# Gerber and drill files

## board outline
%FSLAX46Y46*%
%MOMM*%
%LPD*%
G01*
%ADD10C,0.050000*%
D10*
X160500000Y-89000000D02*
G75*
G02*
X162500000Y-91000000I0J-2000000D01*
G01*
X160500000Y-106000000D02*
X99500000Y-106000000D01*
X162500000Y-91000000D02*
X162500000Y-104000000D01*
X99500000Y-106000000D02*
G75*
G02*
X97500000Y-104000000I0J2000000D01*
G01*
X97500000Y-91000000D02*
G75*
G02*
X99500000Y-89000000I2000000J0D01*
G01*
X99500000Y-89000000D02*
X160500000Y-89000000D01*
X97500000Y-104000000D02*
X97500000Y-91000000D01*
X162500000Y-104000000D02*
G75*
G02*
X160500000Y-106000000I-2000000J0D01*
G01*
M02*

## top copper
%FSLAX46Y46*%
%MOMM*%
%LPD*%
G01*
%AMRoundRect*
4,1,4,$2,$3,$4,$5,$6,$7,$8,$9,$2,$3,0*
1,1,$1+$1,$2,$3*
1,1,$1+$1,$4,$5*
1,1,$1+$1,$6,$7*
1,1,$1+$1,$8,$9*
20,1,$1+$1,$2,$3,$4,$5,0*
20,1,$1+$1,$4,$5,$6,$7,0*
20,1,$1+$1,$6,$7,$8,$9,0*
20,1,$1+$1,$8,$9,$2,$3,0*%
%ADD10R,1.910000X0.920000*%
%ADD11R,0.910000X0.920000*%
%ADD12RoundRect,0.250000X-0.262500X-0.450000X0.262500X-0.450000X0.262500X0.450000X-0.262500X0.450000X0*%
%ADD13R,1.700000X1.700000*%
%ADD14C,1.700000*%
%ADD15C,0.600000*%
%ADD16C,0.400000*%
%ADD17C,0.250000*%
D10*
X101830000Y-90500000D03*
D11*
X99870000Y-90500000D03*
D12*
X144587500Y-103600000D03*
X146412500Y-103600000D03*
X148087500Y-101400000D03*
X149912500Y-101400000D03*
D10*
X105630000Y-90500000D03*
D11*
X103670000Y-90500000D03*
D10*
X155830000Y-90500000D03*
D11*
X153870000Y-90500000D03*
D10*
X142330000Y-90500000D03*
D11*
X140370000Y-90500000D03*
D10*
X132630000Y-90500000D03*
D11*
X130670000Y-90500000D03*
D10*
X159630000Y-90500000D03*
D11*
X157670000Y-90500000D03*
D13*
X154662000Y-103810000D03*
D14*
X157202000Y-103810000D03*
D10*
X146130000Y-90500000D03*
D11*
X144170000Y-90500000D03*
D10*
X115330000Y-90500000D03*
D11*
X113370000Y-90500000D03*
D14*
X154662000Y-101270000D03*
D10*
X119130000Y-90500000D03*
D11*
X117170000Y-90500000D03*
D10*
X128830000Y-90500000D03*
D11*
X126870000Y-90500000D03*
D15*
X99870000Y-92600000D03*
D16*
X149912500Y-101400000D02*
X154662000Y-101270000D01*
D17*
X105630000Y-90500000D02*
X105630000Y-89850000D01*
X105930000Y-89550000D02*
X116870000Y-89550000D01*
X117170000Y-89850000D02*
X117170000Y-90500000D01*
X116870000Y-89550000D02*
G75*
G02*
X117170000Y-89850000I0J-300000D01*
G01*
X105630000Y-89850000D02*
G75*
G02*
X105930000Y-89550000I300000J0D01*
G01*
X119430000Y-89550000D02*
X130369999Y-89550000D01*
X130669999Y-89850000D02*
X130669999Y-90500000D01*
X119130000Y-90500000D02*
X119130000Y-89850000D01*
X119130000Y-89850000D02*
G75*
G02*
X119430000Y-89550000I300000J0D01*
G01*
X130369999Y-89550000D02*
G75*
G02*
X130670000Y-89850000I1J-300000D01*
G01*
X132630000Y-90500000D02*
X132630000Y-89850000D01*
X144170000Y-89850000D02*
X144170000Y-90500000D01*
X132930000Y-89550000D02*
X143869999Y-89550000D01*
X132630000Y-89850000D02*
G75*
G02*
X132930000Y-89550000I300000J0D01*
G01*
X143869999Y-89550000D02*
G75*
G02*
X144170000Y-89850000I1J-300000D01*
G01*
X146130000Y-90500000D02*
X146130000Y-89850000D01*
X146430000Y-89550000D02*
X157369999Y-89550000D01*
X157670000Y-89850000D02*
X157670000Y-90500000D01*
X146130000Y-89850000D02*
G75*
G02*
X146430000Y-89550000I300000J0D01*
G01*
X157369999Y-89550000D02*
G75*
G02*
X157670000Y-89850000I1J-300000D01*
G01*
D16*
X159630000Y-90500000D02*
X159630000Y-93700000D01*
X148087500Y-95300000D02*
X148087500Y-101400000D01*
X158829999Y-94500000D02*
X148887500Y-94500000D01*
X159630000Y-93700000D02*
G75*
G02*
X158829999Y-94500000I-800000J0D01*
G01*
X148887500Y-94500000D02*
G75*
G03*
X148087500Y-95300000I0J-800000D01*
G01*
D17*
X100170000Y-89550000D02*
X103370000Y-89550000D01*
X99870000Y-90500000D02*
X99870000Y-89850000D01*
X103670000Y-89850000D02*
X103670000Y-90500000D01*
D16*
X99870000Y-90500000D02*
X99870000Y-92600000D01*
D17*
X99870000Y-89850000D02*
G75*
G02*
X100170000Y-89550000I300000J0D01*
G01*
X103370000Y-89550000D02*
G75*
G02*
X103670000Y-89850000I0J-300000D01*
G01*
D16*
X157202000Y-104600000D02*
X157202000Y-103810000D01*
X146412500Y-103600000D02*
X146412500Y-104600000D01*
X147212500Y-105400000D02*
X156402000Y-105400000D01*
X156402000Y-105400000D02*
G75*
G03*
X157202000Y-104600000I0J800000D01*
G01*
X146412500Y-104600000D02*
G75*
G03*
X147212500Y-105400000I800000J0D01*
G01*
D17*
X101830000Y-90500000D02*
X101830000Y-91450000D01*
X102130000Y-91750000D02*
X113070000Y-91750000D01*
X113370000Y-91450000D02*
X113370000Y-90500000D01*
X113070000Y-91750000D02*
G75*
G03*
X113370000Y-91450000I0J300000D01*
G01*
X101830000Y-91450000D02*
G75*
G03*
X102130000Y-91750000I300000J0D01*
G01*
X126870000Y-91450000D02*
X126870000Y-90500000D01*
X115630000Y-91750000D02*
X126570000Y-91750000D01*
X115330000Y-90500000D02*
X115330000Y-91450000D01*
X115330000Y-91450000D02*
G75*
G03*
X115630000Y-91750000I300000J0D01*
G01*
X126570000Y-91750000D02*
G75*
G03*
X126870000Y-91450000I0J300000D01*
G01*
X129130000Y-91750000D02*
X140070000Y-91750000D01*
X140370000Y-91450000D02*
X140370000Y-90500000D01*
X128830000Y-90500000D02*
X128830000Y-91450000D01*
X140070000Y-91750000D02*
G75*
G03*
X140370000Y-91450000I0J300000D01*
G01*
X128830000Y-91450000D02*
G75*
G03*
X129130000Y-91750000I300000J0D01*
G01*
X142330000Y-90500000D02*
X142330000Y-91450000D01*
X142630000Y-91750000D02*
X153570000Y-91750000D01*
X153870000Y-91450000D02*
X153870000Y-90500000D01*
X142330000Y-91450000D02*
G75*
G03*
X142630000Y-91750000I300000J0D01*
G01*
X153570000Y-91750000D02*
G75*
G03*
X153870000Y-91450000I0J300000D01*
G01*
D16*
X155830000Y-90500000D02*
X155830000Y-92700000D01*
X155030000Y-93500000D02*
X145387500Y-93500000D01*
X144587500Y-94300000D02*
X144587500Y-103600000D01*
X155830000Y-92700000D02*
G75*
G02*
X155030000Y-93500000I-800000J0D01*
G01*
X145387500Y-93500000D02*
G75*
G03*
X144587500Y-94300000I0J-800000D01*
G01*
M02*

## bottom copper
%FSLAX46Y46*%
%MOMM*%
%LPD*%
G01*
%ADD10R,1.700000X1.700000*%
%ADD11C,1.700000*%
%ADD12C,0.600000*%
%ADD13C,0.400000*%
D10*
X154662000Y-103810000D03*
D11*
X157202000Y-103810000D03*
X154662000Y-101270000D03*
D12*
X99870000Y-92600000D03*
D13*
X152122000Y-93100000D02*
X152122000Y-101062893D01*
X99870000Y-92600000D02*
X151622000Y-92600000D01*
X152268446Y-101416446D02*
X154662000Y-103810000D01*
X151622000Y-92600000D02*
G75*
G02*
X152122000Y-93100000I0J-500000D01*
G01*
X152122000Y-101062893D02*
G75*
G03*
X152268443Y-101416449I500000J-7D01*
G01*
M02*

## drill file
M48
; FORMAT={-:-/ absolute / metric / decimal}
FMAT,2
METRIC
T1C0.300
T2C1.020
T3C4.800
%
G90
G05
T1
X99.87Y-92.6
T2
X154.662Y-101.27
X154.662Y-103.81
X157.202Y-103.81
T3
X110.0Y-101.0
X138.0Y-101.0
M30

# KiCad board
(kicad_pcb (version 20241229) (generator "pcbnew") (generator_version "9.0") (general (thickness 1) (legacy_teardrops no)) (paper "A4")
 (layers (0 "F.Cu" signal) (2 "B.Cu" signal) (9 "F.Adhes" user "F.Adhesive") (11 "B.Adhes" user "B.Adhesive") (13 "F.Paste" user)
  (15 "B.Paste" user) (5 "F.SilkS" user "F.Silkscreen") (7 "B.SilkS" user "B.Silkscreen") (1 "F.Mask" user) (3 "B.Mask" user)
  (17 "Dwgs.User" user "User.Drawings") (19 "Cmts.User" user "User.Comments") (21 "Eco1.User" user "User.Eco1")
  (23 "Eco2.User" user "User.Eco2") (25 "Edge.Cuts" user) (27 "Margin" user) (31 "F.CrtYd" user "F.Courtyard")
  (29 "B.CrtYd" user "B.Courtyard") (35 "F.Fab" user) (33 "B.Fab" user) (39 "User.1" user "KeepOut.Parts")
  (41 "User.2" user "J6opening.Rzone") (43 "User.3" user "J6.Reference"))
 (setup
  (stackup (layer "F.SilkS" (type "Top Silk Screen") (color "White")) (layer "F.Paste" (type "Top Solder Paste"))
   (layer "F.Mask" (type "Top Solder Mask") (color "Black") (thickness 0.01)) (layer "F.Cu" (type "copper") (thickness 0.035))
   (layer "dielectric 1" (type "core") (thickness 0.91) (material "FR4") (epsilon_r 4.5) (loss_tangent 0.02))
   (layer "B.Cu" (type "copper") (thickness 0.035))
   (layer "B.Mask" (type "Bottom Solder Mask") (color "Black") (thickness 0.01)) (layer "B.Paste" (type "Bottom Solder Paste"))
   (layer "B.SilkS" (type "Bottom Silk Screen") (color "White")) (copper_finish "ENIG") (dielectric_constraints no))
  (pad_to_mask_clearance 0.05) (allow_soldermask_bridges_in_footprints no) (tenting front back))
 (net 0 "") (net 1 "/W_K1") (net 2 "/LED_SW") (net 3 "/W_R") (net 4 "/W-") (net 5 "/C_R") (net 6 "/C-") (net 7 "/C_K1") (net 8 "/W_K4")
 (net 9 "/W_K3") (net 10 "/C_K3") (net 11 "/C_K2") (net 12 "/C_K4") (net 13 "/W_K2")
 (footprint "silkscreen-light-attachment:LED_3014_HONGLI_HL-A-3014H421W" (layer "F.Cu") (at 101.1 90.5 180)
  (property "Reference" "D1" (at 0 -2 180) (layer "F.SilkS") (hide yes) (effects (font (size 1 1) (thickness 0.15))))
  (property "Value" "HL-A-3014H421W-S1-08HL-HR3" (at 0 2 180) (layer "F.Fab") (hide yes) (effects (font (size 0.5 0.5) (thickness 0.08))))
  (pad "1" smd rect (at -0.73 0 180) (size 1.91 0.92) (layers "F.Cu" "F.Mask" "F.Paste") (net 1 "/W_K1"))
  (pad "2" smd rect (at 1.23 0 180) (size 0.91 0.92) (layers "F.Cu" "F.Mask" "F.Paste") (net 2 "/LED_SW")))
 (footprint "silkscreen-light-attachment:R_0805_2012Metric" (layer "F.Cu") (at 145.5 103.6)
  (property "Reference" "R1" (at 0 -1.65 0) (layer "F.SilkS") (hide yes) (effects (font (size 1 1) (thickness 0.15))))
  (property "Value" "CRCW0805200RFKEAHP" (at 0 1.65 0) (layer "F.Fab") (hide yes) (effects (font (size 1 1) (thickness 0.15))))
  (pad "1" smd roundrect (at -0.9125 0) (size 1.025 1.4) (layers "F.Cu" "F.Mask" "F.Paste") (roundrect_rratio 0.243902) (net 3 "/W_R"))
  (pad "2" smd roundrect (at 0.9125 0) (size 1.025 1.4) (layers "F.Cu" "F.Mask" "F.Paste") (roundrect_rratio 0.243902) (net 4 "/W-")))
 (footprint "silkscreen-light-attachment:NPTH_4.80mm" (layer "F.Cu") (at 110 101)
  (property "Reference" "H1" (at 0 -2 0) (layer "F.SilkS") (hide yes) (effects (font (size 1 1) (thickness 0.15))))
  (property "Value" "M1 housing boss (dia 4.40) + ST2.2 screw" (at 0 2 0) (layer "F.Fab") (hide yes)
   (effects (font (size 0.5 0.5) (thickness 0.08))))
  (pad "" np_thru_hole circle (at 0 0) (size 4.8 4.8) (drill 4.8) (layers "*.Cu" "*.Mask")))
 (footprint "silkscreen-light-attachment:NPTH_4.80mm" (layer "F.Cu") (at 138 101)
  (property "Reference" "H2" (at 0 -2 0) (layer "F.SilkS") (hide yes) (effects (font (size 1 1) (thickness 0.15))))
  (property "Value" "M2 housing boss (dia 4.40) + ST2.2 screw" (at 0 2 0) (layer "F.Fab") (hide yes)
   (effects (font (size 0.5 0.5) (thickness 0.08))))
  (pad "" np_thru_hole circle (at 0 0) (size 4.8 4.8) (drill 4.8) (layers "*.Cu" "*.Mask")))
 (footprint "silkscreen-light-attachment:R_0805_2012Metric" (layer "F.Cu") (at 149 101.4)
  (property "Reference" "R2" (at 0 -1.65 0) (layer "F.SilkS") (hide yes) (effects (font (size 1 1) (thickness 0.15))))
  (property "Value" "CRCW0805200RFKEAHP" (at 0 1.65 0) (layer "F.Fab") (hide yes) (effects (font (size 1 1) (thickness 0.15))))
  (pad "1" smd roundrect (at -0.9125 0) (size 1.025 1.4) (layers "F.Cu" "F.Mask" "F.Paste") (roundrect_rratio 0.243902) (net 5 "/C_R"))
  (pad "2" smd roundrect (at 0.9125 0) (size 1.025 1.4) (layers "F.Cu" "F.Mask" "F.Paste") (roundrect_rratio 0.243902) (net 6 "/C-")))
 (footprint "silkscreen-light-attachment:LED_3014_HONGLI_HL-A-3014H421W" (layer "F.Cu") (at 104.9 90.5 180)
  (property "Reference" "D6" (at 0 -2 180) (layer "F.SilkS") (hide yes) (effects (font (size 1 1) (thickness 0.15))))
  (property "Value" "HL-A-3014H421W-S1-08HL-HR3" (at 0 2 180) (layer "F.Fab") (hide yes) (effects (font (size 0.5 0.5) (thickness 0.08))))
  (pad "1" smd rect (at -0.73 0 180) (size 1.91 0.92) (layers "F.Cu" "F.Mask" "F.Paste") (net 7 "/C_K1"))
  (pad "2" smd rect (at 1.23 0 180) (size 0.91 0.92) (layers "F.Cu" "F.Mask" "F.Paste") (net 2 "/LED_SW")))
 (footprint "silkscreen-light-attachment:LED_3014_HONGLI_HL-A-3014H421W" (layer "F.Cu") (at 155.1 90.5 180)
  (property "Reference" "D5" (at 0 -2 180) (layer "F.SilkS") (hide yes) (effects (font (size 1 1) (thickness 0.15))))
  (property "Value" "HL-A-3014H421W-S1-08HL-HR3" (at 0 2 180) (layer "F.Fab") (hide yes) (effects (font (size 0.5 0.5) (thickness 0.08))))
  (pad "1" smd rect (at -0.73 0 180) (size 1.91 0.92) (layers "F.Cu" "F.Mask" "F.Paste") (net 3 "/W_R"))
  (pad "2" smd rect (at 1.23 0 180) (size 0.91 0.92) (layers "F.Cu" "F.Mask" "F.Paste") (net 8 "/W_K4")))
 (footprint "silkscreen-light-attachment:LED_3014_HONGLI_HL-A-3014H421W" (layer "F.Cu") (at 141.6 90.5 180)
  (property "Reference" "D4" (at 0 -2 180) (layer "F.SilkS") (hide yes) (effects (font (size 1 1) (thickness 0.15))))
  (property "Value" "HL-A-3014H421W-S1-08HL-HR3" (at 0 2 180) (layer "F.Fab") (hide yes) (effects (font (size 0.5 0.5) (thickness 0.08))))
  (pad "1" smd rect (at -0.73 0 180) (size 1.91 0.92) (layers "F.Cu" "F.Mask" "F.Paste") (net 8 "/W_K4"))
  (pad "2" smd rect (at 1.23 0 180) (size 0.91 0.92) (layers "F.Cu" "F.Mask" "F.Paste") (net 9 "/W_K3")))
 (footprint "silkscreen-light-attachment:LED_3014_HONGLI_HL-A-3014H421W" (layer "F.Cu") (at 131.9 90.5 180)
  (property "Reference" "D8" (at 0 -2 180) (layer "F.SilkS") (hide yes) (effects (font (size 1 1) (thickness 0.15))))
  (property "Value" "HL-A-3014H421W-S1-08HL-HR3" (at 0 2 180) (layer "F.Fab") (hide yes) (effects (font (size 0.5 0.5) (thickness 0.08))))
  (pad "1" smd rect (at -0.73 0 180) (size 1.91 0.92) (layers "F.Cu" "F.Mask" "F.Paste") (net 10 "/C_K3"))
  (pad "2" smd rect (at 1.23 0 180) (size 0.91 0.92) (layers "F.Cu" "F.Mask" "F.Paste") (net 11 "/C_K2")))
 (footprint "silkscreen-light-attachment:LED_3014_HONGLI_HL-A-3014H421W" (layer "F.Cu") (at 158.9 90.5 180)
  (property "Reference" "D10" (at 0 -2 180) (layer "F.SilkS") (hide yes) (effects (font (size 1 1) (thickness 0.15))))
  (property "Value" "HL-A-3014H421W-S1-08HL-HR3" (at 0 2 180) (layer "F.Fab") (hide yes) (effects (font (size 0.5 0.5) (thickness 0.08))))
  (pad "1" smd rect (at -0.73 0 180) (size 1.91 0.92) (layers "F.Cu" "F.Mask" "F.Paste") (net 5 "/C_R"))
  (pad "2" smd rect (at 1.23 0 180) (size 0.91 0.92) (layers "F.Cu" "F.Mask" "F.Paste") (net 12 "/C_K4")))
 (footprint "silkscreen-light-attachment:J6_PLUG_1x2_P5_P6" (layer "F.Cu") (at 155.932 103.81)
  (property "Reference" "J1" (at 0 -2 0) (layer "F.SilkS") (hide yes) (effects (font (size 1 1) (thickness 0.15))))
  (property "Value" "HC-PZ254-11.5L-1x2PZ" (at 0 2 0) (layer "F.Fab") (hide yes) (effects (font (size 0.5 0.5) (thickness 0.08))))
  (pad "5" thru_hole rect (at -1.27 0) (size 1.7 1.7) (drill 1.02) (layers "*.Cu" "*.Mask") (remove_unused_layers no) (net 2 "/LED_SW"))
  (pad "6" thru_hole circle (at 1.27 0) (size 1.7 1.7) (drill 1.02) (layers "*.Cu" "*.Mask") (remove_unused_layers no) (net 4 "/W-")))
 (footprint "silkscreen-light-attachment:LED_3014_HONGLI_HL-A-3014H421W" (layer "F.Cu") (at 145.4 90.5 180)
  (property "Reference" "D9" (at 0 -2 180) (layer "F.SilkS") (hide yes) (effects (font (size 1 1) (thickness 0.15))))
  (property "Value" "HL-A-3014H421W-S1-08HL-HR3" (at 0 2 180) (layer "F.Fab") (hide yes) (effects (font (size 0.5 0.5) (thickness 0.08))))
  (pad "1" smd rect (at -0.73 0 180) (size 1.91 0.92) (layers "F.Cu" "F.Mask" "F.Paste") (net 12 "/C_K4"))
  (pad "2" smd rect (at 1.23 0 180) (size 0.91 0.92) (layers "F.Cu" "F.Mask" "F.Paste") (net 10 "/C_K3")))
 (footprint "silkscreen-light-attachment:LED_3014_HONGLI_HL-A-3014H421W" (layer "F.Cu") (at 114.6 90.5 180)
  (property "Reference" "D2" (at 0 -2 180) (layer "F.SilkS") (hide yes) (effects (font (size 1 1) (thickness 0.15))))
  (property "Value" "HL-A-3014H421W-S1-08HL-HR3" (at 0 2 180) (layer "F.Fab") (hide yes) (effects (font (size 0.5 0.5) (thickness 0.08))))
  (pad "1" smd rect (at -0.73 0 180) (size 1.91 0.92) (layers "F.Cu" "F.Mask" "F.Paste") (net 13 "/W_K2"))
  (pad "2" smd rect (at 1.23 0 180) (size 0.91 0.92) (layers "F.Cu" "F.Mask" "F.Paste") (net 1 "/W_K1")))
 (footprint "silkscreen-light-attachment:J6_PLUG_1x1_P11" (layer "F.Cu") (at 154.662 101.27)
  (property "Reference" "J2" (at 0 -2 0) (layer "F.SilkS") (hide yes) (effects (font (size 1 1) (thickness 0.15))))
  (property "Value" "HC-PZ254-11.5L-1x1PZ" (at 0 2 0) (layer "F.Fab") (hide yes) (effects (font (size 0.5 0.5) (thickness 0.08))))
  (pad "11" thru_hole circle (at 0 0) (size 1.7 1.7) (drill 1.02) (layers "*.Cu" "*.Mask") (remove_unused_layers no) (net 6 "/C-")))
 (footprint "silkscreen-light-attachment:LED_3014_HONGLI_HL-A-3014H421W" (layer "F.Cu") (at 118.4 90.5 180)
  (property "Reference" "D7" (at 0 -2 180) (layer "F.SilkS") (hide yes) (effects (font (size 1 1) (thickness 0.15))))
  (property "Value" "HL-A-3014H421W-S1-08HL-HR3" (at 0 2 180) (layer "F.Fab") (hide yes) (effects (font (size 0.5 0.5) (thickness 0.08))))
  (pad "1" smd rect (at -0.73 0 180) (size 1.91 0.92) (layers "F.Cu" "F.Mask" "F.Paste") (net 11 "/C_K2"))
  (pad "2" smd rect (at 1.23 0 180) (size 0.91 0.92) (layers "F.Cu" "F.Mask" "F.Paste") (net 7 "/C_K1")))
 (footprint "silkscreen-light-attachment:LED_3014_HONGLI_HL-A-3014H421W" (layer "F.Cu") (at 128.1 90.5 180)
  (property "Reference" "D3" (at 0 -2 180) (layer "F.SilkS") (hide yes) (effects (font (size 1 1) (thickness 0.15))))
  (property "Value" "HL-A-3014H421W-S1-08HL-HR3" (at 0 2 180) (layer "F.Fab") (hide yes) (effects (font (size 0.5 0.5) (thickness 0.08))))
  (pad "1" smd rect (at -0.73 0 180) (size 1.91 0.92) (layers "F.Cu" "F.Mask" "F.Paste") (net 9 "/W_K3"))
  (pad "2" smd rect (at 1.23 0 180) (size 0.91 0.92) (layers "F.Cu" "F.Mask" "F.Paste") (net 13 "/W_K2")))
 (gr_arc (start 160.5 89) (mid 161.914213 89.585786) (end 162.5 91) (stroke (width 0.05) (type default)) (layer "Edge.Cuts"))
 (gr_line (start 160.5 106) (end 99.5 106) (stroke (width 0.05) (type default)) (layer "Edge.Cuts"))
 (gr_line (start 162.5 91) (end 162.5 104) (stroke (width 0.05) (type default)) (layer "Edge.Cuts"))
 (gr_arc (start 99.5 106) (mid 98.085786 105.414213) (end 97.5 104) (stroke (width 0.05) (type default)) (layer "Edge.Cuts"))
 (gr_arc (start 97.5 91) (mid 98.085786 89.585786) (end 99.5 89) (stroke (width 0.05) (type default)) (layer "Edge.Cuts"))
 (gr_line (start 99.5 89) (end 160.5 89) (stroke (width 0.05) (type default)) (layer "Edge.Cuts"))
 (gr_line (start 97.5 104) (end 97.5 91) (stroke (width 0.05) (type default)) (layer "Edge.Cuts"))
 (gr_arc (start 162.5 104) (mid 161.914213 105.414213) (end 160.5 106) (stroke (width 0.05) (type default)) (layer "Edge.Cuts"))
 (segment (start 149.9125 101.4) (end 154.662 101.27) (width 0.4) (layer "F.Cu") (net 6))
 (segment (start 105.63 90.5) (end 105.63 89.85) (width 0.25) (layer "F.Cu") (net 7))
 (segment (start 105.93 89.55) (end 116.87 89.55) (width 0.25) (layer "F.Cu") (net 7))
 (segment (start 117.17 89.85) (end 117.17 90.5) (width 0.25) (layer "F.Cu") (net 7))
 (arc (start 116.87 89.55) (mid 117.082132 89.637867) (end 117.17 89.85) (width 0.25) (layer "F.Cu") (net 7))
 (arc (start 105.63 89.85) (mid 105.717867 89.637867) (end 105.93 89.55) (width 0.25) (layer "F.Cu") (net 7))
 (segment (start 119.43 89.55) (end 130.369999 89.55) (width 0.25) (layer "F.Cu") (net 11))
 (segment (start 130.669999 89.85) (end 130.669999 90.5) (width 0.25) (layer "F.Cu") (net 11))
 (segment (start 119.13 90.5) (end 119.13 89.85) (width 0.25) (layer "F.Cu") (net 11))
 (arc (start 119.13 89.85) (mid 119.217867 89.637867) (end 119.43 89.55) (width 0.25) (layer "F.Cu") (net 11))
 (arc (start 130.369999 89.55) (mid 130.582132 89.637867) (end 130.669999 89.85) (width 0.25) (layer "F.Cu") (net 11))
 (segment (start 132.63 90.5) (end 132.63 89.85) (width 0.25) (layer "F.Cu") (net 10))
 (segment (start 144.17 89.85) (end 144.17 90.5) (width 0.25) (layer "F.Cu") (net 10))
 (segment (start 132.93 89.55) (end 143.869999 89.55) (width 0.25) (layer "F.Cu") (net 10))
 (arc (start 132.63 89.85) (mid 132.717867 89.637867) (end 132.93 89.55) (width 0.25) (layer "F.Cu") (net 10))
 (arc (start 143.869999 89.55) (mid 144.082132 89.637867) (end 144.17 89.85) (width 0.25) (layer "F.Cu") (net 10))
 (segment (start 146.13 90.5) (end 146.13 89.85) (width 0.25) (layer "F.Cu") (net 12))
 (segment (start 146.43 89.55) (end 157.369999 89.55) (width 0.25) (layer "F.Cu") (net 12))
 (segment (start 157.67 89.85) (end 157.67 90.5) (width 0.25) (layer "F.Cu") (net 12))
 (arc (start 146.13 89.85) (mid 146.217867 89.637867) (end 146.43 89.55) (width 0.25) (layer "F.Cu") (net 12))
 (arc (start 157.369999 89.55) (mid 157.582132 89.637867) (end 157.67 89.85) (width 0.25) (layer "F.Cu") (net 12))
 (segment (start 159.63 90.5) (end 159.63 93.7) (width 0.4) (layer "F.Cu") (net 5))
 (segment (start 148.0875 95.3) (end 148.0875 101.4) (width 0.4) (layer "F.Cu") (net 5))
 (segment (start 158.829999 94.5) (end 148.8875 94.5) (width 0.4) (layer "F.Cu") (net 5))
 (arc (start 159.63 93.7) (mid 159.395685 94.265685) (end 158.829999 94.5) (width 0.4) (layer "F.Cu") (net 5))
 (arc (start 148.8875 94.5) (mid 148.321814 94.734314) (end 148.0875 95.3) (width 0.4) (layer "F.Cu") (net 5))
 (segment (start 100.17 89.55) (end 103.37 89.55) (width 0.25) (layer "F.Cu") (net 2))
 (segment (start 99.87 90.5) (end 99.87 89.85) (width 0.25) (layer "F.Cu") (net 2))
 (segment (start 103.67 89.85) (end 103.67 90.5) (width 0.25) (layer "F.Cu") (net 2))
 (segment (start 99.87 90.5) (end 99.87 92.6) (width 0.4) (layer "F.Cu") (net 2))
 (via (at 99.87 92.6) (size 0.6) (drill 0.3) (layers "F.Cu" "B.Cu") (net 2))
 (arc (start 99.87 89.85) (mid 99.957867 89.637867) (end 100.17 89.55) (width 0.25) (layer "F.Cu") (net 2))
 (arc (start 103.37 89.55) (mid 103.582132 89.637867) (end 103.67 89.85) (width 0.25) (layer "F.Cu") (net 2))
 (segment (start 152.122 93.1) (end 152.122 101.062893) (width 0.4) (layer "B.Cu") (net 2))
 (segment (start 99.87 92.6) (end 151.622 92.6) (width 0.4) (layer "B.Cu") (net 2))
 (segment (start 152.268446 101.416446) (end 154.662 103.81) (width 0.4) (layer "B.Cu") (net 2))
 (arc (start 151.622 92.6) (mid 151.975553 92.746446) (end 152.122 93.1) (width 0.4) (layer "B.Cu") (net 2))
 (arc (start 152.122 101.062893) (mid 152.16006 101.254234) (end 152.268446 101.416446) (width 0.4) (layer "B.Cu") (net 2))
 (segment (start 157.202 104.6) (end 157.202 103.81) (width 0.4) (layer "F.Cu") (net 4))
 (segment (start 146.4125 103.6) (end 146.4125 104.6) (width 0.4) (layer "F.Cu") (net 4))
 (segment (start 147.2125 105.4) (end 156.402 105.4) (width 0.4) (layer "F.Cu") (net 4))
 (arc (start 156.402 105.4) (mid 156.967685 105.165685) (end 157.202 104.6) (width 0.4) (layer "F.Cu") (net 4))
 (arc (start 146.4125 104.6) (mid 146.646814 105.165685) (end 147.2125 105.4) (width 0.4) (layer "F.Cu") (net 4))
 (segment (start 101.83 90.5) (end 101.83 91.45) (width 0.25) (layer "F.Cu") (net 1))
 (segment (start 102.13 91.75) (end 113.07 91.75) (width 0.25) (layer "F.Cu") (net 1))
 (segment (start 113.37 91.45) (end 113.37 90.5) (width 0.25) (layer "F.Cu") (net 1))
 (arc (start 113.07 91.75) (mid 113.282132 91.662132) (end 113.37 91.45) (width 0.25) (layer "F.Cu") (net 1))
 (arc (start 101.83 91.45) (mid 101.917867 91.662132) (end 102.13 91.75) (width 0.25) (layer "F.Cu") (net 1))
 (segment (start 126.87 91.45) (end 126.87 90.5) (width 0.25) (layer "F.Cu") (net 13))
 (segment (start 115.63 91.75) (end 126.57 91.75) (width 0.25) (layer "F.Cu") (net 13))
 (segment (start 115.33 90.5) (end 115.33 91.45) (width 0.25) (layer "F.Cu") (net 13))
 (arc (start 115.33 91.45) (mid 115.417867 91.662132) (end 115.63 91.75) (width 0.25) (layer "F.Cu") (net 13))
 (arc (start 126.57 91.75) (mid 126.782132 91.662132) (end 126.87 91.45) (width 0.25) (layer "F.Cu") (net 13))
 (segment (start 129.13 91.75) (end 140.07 91.75) (width 0.25) (layer "F.Cu") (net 9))
 (segment (start 140.37 91.45) (end 140.37 90.5) (width 0.25) (layer "F.Cu") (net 9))
 (segment (start 128.83 90.5) (end 128.83 91.45) (width 0.25) (layer "F.Cu") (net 9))
 (arc (start 140.07 91.75) (mid 140.282132 91.662132) (end 140.37 91.45) (width 0.25) (layer "F.Cu") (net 9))
 (arc (start 128.83 91.45) (mid 128.917867 91.662132) (end 129.13 91.75) (width 0.25) (layer "F.Cu") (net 9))
 (segment (start 142.33 90.5) (end 142.33 91.45) (width 0.25) (layer "F.Cu") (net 8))
 (segment (start 142.63 91.75) (end 153.57 91.75) (width 0.25) (layer "F.Cu") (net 8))
 (segment (start 153.87 91.45) (end 153.87 90.5) (width 0.25) (layer "F.Cu") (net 8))
 (arc (start 142.33 91.45) (mid 142.417867 91.662132) (end 142.63 91.75) (width 0.25) (layer "F.Cu") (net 8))
 (arc (start 153.57 91.75) (mid 153.782132 91.662132) (end 153.87 91.45) (width 0.25) (layer "F.Cu") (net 8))
 (segment (start 155.83 90.5) (end 155.83 92.7) (width 0.4) (layer "F.Cu") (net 3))
 (segment (start 155.03 93.5) (end 145.3875 93.5) (width 0.4) (layer "F.Cu") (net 3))
 (segment (start 144.5875 94.3) (end 144.5875 103.6) (width 0.4) (layer "F.Cu") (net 3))
 (arc (start 155.83 92.7) (mid 155.595685 93.265685) (end 155.03 93.5) (width 0.4) (layer "F.Cu") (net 3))
 (arc (start 145.3875 93.5) (mid 144.821814 93.734314) (end 144.5875 94.3) (width 0.4) (layer "F.Cu") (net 3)))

